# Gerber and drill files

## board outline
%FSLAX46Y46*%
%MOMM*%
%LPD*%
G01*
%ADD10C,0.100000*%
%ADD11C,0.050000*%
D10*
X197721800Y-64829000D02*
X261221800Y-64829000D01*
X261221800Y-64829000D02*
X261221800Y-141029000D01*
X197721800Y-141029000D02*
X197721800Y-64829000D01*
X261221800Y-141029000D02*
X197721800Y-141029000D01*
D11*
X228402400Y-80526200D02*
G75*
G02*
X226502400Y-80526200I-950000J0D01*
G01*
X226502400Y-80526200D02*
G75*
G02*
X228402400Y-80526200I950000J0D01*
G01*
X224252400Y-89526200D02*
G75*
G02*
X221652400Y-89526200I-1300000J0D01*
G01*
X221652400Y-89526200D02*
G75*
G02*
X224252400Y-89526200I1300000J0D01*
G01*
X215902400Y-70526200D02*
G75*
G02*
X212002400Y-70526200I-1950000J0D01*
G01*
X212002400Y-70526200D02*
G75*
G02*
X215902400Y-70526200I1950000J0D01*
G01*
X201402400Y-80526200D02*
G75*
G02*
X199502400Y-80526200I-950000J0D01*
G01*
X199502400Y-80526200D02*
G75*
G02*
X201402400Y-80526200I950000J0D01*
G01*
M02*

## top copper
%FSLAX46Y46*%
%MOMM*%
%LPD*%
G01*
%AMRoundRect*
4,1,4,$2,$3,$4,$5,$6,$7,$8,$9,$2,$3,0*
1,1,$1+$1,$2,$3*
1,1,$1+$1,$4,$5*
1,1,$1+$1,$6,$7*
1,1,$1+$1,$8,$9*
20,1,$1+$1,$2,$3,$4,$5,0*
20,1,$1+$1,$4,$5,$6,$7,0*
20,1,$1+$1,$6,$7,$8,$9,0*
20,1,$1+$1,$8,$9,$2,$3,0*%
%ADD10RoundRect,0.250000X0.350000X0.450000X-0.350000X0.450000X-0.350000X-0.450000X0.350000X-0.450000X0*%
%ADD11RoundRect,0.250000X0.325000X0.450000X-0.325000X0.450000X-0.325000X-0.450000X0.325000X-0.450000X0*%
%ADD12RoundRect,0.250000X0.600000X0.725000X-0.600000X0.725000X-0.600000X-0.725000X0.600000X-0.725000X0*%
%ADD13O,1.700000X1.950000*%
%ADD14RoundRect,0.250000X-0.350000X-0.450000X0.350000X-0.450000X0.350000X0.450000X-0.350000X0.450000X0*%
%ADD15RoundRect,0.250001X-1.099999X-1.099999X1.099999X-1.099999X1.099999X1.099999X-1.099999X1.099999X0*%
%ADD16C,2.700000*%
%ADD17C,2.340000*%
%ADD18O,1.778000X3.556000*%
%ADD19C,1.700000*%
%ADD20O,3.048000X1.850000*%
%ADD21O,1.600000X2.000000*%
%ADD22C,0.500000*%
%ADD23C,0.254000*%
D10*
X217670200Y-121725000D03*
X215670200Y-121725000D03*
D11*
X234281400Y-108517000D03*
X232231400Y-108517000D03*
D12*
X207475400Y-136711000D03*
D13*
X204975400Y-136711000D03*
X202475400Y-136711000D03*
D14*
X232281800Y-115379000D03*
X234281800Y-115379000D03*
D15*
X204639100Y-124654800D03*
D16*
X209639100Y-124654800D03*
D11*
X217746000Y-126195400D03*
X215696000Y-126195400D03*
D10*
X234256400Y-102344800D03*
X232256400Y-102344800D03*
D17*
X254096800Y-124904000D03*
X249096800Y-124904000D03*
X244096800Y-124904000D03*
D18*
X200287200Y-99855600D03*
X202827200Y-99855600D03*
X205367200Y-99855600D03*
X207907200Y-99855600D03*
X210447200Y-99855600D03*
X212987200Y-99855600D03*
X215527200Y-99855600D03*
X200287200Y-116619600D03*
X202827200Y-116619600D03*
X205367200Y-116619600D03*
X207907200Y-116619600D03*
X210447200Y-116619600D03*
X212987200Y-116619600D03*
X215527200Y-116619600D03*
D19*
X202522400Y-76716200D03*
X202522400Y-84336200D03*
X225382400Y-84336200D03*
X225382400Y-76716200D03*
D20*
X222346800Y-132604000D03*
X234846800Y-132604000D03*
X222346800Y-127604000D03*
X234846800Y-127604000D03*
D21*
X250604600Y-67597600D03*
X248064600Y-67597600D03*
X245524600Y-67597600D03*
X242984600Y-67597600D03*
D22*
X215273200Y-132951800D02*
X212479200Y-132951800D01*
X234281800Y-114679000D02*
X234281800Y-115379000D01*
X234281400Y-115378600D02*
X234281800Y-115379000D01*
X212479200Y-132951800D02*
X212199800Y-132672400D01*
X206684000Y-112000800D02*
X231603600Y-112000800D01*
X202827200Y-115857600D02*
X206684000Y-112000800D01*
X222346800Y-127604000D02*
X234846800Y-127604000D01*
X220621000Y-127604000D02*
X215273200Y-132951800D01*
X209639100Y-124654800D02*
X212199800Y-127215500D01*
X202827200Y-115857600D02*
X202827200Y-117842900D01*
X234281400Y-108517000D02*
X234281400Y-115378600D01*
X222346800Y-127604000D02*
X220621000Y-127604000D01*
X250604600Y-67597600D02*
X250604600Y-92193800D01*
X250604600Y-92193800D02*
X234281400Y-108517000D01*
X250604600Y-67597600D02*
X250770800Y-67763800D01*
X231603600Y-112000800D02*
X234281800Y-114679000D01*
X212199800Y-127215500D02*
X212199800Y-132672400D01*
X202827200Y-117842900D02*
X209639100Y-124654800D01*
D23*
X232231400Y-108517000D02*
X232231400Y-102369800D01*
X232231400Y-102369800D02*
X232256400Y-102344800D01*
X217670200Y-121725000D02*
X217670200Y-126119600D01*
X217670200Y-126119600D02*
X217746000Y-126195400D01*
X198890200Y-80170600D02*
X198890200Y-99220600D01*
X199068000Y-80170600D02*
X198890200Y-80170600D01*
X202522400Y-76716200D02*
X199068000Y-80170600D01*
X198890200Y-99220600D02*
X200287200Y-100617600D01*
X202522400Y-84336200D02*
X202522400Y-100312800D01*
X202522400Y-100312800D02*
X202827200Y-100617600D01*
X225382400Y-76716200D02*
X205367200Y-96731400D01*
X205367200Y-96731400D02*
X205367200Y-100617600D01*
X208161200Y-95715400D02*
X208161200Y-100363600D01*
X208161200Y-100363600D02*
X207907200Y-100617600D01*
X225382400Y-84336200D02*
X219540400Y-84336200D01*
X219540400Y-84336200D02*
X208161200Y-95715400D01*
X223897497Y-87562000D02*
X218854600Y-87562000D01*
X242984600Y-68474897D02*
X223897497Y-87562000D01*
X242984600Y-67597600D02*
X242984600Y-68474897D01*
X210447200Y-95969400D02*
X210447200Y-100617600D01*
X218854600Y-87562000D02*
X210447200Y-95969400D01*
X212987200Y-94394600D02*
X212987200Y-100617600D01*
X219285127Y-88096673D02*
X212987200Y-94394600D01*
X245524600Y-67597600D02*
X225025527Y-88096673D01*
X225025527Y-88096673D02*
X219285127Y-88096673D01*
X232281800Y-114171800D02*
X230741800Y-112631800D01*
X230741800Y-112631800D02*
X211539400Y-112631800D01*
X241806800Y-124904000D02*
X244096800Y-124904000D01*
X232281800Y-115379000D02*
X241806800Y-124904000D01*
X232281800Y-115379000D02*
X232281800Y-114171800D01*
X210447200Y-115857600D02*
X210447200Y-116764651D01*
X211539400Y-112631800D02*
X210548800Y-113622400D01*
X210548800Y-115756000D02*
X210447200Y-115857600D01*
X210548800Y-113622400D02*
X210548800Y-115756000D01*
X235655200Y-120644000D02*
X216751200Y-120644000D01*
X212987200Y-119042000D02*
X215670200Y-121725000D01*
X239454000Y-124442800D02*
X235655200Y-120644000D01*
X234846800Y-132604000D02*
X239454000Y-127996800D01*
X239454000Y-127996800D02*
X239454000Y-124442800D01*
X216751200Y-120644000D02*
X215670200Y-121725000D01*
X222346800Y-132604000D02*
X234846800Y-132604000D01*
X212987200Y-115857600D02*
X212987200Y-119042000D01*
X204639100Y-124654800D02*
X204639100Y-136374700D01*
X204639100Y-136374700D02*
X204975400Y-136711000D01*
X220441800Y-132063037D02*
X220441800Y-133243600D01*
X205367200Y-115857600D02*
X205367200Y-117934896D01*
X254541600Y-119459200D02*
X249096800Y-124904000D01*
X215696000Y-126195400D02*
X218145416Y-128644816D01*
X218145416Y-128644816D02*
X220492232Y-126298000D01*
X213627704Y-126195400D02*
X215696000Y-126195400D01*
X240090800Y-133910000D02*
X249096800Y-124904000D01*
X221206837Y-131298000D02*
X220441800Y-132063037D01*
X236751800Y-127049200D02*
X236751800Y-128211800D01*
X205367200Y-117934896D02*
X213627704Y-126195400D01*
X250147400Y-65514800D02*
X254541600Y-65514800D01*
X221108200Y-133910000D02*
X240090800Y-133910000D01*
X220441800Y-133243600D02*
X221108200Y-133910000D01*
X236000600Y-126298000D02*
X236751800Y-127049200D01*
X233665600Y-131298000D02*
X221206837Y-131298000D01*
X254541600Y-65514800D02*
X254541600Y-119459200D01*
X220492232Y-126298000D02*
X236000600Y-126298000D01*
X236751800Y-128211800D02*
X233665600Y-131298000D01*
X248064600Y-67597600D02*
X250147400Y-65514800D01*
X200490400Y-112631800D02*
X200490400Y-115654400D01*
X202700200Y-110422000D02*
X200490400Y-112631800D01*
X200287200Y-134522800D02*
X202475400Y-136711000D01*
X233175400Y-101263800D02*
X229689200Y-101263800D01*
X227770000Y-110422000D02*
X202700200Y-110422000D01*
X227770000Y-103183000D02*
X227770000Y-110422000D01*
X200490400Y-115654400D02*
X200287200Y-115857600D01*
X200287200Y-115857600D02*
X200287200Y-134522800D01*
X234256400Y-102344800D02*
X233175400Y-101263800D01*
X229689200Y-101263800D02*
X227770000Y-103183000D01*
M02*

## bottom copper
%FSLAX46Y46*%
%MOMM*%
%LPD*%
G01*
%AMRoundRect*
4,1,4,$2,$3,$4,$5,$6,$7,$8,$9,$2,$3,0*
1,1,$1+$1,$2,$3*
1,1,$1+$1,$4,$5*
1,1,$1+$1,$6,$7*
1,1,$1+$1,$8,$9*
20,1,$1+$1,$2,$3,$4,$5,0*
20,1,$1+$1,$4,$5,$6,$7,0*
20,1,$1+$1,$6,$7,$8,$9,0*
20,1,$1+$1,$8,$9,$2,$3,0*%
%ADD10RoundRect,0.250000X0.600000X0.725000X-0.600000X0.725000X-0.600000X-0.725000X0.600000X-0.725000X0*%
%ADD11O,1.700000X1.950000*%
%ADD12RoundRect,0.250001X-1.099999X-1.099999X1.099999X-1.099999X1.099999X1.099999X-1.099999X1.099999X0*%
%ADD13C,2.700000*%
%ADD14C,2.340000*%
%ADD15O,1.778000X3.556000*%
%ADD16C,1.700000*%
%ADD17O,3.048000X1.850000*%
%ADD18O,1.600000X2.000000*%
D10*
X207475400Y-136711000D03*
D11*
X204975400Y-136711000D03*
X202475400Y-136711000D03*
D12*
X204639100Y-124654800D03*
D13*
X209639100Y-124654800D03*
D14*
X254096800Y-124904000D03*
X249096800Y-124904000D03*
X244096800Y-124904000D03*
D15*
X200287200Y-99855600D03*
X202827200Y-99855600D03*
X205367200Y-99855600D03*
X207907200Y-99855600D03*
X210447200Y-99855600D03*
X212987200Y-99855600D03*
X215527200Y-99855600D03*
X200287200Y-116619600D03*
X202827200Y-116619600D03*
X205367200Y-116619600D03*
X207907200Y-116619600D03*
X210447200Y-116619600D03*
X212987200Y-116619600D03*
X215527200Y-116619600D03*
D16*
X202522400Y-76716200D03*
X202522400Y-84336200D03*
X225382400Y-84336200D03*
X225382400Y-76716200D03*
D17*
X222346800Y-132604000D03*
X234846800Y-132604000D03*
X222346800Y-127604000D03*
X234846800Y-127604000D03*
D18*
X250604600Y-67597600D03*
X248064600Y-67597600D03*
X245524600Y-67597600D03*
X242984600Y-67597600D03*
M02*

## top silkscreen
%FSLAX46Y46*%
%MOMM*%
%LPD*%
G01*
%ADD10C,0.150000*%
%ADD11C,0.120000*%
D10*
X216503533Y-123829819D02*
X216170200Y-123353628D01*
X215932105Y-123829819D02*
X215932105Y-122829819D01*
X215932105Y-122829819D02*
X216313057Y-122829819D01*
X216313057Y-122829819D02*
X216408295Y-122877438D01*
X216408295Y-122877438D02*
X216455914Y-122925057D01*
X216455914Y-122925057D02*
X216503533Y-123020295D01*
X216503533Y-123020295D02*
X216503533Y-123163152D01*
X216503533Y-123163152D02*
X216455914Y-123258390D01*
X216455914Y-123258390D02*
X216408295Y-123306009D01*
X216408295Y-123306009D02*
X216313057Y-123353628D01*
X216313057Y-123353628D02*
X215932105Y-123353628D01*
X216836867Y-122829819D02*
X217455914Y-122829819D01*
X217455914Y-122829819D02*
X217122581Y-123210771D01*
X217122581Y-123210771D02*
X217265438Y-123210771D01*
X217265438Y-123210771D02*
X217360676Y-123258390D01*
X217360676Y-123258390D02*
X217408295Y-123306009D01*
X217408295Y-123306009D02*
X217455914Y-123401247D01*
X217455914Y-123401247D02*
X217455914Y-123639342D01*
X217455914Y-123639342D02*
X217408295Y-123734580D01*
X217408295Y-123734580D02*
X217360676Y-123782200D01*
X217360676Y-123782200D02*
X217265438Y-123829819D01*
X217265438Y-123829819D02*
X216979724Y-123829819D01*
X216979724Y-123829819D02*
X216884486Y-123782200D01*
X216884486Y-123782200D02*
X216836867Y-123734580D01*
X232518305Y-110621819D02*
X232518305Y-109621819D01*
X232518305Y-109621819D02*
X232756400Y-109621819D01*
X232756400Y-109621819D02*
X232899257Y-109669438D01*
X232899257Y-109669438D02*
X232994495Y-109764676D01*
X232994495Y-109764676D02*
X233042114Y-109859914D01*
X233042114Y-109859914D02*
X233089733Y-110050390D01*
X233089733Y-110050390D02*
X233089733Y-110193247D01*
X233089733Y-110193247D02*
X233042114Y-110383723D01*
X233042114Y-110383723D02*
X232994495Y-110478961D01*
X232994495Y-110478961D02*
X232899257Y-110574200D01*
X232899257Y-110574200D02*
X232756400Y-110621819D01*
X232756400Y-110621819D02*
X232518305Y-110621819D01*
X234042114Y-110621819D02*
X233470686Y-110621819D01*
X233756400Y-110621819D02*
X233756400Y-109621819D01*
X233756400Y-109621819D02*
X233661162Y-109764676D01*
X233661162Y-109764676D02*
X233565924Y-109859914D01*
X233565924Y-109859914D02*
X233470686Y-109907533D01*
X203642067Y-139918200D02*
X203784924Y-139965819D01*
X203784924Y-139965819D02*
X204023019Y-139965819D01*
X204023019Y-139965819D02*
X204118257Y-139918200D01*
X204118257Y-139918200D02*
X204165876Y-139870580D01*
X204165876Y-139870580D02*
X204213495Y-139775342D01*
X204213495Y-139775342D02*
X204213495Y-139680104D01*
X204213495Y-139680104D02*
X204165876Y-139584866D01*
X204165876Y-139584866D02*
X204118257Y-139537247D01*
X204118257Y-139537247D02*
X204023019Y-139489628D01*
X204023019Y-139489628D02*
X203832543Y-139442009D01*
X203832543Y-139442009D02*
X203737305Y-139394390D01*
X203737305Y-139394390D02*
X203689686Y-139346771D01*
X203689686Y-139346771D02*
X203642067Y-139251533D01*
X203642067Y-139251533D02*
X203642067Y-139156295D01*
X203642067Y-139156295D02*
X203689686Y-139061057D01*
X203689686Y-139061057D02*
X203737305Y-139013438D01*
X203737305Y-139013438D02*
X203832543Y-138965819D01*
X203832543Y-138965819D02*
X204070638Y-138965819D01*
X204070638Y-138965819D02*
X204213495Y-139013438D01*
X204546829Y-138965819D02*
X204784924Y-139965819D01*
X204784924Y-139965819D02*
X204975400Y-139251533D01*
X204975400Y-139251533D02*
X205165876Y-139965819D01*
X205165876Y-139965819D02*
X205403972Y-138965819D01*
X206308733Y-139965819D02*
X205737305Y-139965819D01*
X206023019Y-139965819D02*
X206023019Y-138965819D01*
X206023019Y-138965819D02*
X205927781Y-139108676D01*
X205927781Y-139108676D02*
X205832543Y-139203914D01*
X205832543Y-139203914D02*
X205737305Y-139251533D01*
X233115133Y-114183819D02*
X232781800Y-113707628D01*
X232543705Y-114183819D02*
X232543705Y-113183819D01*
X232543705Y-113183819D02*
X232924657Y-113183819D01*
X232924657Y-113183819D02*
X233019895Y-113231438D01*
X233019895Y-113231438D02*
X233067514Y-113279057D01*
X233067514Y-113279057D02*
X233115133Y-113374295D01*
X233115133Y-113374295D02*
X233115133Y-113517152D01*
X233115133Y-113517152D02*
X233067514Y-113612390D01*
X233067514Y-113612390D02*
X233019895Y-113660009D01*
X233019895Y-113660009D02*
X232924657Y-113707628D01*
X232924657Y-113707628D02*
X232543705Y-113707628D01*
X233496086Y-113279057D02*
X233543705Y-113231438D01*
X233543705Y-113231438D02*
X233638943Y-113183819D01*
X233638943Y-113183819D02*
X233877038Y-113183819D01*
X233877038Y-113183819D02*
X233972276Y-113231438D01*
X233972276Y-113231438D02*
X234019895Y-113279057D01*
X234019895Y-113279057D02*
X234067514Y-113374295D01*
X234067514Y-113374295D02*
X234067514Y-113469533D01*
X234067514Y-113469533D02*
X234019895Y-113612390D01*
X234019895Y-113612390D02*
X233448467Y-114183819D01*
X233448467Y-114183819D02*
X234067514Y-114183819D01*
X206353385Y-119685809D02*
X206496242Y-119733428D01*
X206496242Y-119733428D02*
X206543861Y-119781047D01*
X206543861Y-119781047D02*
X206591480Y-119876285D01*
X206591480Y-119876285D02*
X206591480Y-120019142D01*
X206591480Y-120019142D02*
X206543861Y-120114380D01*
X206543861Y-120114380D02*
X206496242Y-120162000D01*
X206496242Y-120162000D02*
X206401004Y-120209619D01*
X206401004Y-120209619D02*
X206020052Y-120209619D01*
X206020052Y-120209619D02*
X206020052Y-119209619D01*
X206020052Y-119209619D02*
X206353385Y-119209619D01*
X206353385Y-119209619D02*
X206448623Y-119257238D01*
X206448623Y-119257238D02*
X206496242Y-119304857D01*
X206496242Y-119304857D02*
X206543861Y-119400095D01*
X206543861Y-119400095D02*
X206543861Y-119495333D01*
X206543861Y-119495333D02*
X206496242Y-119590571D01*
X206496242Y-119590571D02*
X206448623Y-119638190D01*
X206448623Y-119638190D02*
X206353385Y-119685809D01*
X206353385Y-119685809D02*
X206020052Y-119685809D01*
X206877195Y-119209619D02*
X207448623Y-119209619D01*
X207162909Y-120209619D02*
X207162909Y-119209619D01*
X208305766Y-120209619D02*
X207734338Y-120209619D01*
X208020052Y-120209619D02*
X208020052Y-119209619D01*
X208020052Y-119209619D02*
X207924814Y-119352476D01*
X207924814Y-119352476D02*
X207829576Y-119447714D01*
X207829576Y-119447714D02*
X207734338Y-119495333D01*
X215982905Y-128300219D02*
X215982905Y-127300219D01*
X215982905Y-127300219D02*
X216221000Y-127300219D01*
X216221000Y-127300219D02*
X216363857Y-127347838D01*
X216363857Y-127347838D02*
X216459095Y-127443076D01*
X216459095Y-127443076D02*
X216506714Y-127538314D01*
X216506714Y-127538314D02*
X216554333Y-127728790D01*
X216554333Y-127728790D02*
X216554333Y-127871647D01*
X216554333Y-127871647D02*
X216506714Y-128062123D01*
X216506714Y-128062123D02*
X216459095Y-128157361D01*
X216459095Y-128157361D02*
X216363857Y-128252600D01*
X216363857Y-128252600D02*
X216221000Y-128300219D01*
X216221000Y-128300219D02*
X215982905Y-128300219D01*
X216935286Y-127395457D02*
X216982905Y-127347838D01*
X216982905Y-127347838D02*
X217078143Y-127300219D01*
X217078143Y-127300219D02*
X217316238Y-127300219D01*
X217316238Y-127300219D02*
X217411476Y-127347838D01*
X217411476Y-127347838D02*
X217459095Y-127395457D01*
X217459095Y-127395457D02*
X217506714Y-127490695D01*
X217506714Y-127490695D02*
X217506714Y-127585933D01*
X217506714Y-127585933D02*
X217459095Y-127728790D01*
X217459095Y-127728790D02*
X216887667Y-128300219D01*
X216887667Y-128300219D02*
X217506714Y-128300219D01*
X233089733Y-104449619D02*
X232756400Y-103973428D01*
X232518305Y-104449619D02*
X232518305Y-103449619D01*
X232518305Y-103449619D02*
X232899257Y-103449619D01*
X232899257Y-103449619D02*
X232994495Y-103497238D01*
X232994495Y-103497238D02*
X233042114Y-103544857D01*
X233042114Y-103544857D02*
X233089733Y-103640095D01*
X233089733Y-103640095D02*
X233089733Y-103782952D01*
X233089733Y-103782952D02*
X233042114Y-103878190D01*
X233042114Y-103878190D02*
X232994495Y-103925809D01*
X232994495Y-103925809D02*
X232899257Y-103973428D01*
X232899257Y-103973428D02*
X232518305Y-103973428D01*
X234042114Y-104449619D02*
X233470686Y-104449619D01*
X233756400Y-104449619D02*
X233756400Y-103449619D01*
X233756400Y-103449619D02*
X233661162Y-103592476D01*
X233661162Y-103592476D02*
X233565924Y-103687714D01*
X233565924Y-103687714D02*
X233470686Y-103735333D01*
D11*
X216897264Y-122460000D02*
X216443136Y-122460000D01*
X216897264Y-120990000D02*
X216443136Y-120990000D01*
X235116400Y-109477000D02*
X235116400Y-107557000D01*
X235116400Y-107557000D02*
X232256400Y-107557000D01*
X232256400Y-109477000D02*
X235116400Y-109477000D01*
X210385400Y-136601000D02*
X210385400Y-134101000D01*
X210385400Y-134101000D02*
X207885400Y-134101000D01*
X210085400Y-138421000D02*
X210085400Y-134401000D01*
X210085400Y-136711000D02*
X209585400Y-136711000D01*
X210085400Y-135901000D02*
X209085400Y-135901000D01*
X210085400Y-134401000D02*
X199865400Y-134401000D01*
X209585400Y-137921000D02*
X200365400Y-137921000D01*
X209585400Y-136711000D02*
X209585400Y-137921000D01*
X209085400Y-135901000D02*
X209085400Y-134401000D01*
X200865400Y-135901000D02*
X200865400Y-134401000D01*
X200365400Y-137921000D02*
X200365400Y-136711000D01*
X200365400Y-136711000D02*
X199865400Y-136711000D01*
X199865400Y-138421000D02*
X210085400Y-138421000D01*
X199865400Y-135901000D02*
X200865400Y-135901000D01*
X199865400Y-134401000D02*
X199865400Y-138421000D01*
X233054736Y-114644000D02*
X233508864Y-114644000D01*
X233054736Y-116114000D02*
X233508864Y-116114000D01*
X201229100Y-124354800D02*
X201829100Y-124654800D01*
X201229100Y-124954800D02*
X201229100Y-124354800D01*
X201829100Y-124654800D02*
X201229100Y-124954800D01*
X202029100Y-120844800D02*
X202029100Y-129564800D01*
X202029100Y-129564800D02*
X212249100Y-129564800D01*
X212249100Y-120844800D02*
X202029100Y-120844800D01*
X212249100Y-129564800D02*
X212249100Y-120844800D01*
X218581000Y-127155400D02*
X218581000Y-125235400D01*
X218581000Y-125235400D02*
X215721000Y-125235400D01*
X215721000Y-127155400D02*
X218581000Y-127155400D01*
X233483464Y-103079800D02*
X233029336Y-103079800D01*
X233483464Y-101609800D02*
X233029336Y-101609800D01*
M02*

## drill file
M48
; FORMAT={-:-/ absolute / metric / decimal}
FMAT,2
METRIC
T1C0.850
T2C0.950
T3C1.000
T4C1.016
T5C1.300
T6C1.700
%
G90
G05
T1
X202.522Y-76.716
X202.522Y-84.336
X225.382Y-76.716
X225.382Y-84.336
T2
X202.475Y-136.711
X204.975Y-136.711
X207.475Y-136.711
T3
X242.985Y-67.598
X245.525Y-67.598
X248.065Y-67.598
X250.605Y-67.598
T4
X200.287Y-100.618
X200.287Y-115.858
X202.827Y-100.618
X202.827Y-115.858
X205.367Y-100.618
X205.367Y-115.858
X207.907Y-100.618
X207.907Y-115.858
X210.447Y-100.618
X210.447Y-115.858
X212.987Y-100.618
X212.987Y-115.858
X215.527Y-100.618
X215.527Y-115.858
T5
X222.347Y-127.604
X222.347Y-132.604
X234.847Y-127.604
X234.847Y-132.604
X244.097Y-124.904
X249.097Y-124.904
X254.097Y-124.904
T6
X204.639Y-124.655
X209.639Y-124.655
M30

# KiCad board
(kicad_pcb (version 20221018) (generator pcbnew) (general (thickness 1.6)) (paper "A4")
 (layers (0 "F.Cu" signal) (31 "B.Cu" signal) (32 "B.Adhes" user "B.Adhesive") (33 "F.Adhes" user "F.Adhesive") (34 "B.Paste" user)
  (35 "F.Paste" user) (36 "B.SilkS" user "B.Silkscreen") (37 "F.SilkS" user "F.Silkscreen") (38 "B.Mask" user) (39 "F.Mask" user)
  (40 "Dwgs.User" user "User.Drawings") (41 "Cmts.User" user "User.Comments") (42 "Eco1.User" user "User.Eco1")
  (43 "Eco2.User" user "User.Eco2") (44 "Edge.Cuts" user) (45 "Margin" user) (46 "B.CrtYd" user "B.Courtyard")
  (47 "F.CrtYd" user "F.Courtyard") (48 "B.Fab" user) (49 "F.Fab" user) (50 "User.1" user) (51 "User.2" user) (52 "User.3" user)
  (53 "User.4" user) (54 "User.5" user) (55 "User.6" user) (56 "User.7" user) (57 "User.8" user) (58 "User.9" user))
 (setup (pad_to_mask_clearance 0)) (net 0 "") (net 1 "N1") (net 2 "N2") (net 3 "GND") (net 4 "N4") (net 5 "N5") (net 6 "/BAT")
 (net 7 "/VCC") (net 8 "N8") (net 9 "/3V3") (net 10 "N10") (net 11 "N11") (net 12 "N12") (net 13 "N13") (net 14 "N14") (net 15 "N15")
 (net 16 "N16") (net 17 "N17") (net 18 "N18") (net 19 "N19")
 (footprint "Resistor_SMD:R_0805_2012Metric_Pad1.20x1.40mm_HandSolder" (layer "F.Cu") (at 216.6702 121.725 180)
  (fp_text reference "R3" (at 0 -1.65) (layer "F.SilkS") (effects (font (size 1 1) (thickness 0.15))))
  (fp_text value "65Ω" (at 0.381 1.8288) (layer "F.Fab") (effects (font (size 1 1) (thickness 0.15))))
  (fp_line (start -0.227064 -0.735) (end 0.227064 -0.735) (stroke (width 0.12) (type solid)) (layer "F.SilkS"))
  (fp_line (start -0.227064 0.735) (end 0.227064 0.735) (stroke (width 0.12) (type solid)) (layer "F.SilkS"))
  (pad "1" smd roundrect (at -1 0 180) (size 1.2 1.4) (layers "F.Cu" "F.Paste" "F.Mask") (roundrect_rratio 0.208333) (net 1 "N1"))
  (pad "2" smd roundrect (at 1 0 180) (size 1.2 1.4) (layers "F.Cu" "F.Paste" "F.Mask") (roundrect_rratio 0.208333) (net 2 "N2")))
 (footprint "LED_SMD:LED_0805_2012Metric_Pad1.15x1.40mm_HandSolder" (layer "F.Cu") (at 233.2564 108.517 180)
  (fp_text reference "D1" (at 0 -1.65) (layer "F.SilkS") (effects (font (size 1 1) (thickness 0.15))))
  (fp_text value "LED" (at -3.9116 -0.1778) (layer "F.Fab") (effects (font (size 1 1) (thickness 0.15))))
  (fp_line (start -1.86 -0.96) (end -1.86 0.96) (stroke (width 0.12) (type solid)) (layer "F.SilkS"))
  (fp_line (start -1.86 0.96) (end 1 0.96) (stroke (width 0.12) (type solid)) (layer "F.SilkS"))
  (fp_line (start 1 -0.96) (end -1.86 -0.96) (stroke (width 0.12) (type solid)) (layer "F.SilkS"))
  (pad "1" smd roundrect (at -1.025 0 180) (size 1.15 1.4) (layers "F.Cu" "F.Paste" "F.Mask") (roundrect_rratio 0.217391) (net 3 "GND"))
  (pad "2" smd roundrect (at 1.025 0 180) (size 1.15 1.4) (layers "F.Cu" "F.Paste" "F.Mask") (roundrect_rratio 0.217391) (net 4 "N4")))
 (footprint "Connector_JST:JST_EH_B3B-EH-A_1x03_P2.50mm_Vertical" (layer "F.Cu") (at 207.4754 136.711 180)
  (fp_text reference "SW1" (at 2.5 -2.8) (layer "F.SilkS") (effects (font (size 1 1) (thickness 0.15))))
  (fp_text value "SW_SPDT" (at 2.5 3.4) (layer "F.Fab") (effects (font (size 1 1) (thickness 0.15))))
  (fp_line (start -2.91 0.11) (end -2.91 2.61) (stroke (width 0.12) (type solid)) (layer "F.SilkS"))
  (fp_line (start -2.91 2.61) (end -0.41 2.61) (stroke (width 0.12) (type solid)) (layer "F.SilkS"))
  (fp_line (start -2.61 -1.71) (end -2.61 2.31) (stroke (width 0.12) (type solid)) (layer "F.SilkS"))
  (fp_line (start -2.61 0) (end -2.11 0) (stroke (width 0.12) (type solid)) (layer "F.SilkS"))
  (fp_line (start -2.61 0.81) (end -1.61 0.81) (stroke (width 0.12) (type solid)) (layer "F.SilkS"))
  (fp_line (start -2.61 2.31) (end 7.61 2.31) (stroke (width 0.12) (type solid)) (layer "F.SilkS"))
  (fp_line (start -2.11 -1.21) (end 7.11 -1.21) (stroke (width 0.12) (type solid)) (layer "F.SilkS"))
  (fp_line (start -2.11 0) (end -2.11 -1.21) (stroke (width 0.12) (type solid)) (layer "F.SilkS"))
  (fp_line (start -1.61 0.81) (end -1.61 2.31) (stroke (width 0.12) (type solid)) (layer "F.SilkS"))
  (fp_line (start 6.61 0.81) (end 6.61 2.31) (stroke (width 0.12) (type solid)) (layer "F.SilkS"))
  (fp_line (start 7.11 -1.21) (end 7.11 0) (stroke (width 0.12) (type solid)) (layer "F.SilkS"))
  (fp_line (start 7.11 0) (end 7.61 0) (stroke (width 0.12) (type solid)) (layer "F.SilkS"))
  (fp_line (start 7.61 -1.71) (end -2.61 -1.71) (stroke (width 0.12) (type solid)) (layer "F.SilkS"))
  (fp_line (start 7.61 0.81) (end 6.61 0.81) (stroke (width 0.12) (type solid)) (layer "F.SilkS"))
  (fp_line (start 7.61 2.31) (end 7.61 -1.71) (stroke (width 0.12) (type solid)) (layer "F.SilkS"))
  (pad "1" thru_hole roundrect (at 0 0 180) (size 1.7 1.95) (drill 0.95) (layers "*.Cu" "*.Mask") (roundrect_rratio 0.147059) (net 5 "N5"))
  (pad "2" thru_hole oval (at 2.5 0 180) (size 1.7 1.95) (drill 0.95) (layers "*.Cu" "*.Mask") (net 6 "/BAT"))
  (pad "3" thru_hole oval (at 5 0 180) (size 1.7 1.95) (drill 0.95) (layers "*.Cu" "*.Mask") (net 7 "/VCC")))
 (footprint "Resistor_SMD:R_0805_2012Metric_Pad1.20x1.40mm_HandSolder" (layer "F.Cu") (at 233.2818 115.379)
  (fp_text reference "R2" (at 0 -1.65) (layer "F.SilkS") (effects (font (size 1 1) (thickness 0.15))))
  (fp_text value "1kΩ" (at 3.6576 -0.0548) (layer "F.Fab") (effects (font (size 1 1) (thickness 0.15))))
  (fp_line (start -0.227064 -0.735) (end 0.227064 -0.735) (stroke (width 0.12) (type solid)) (layer "F.SilkS"))
  (fp_line (start -0.227064 0.735) (end 0.227064 0.735) (stroke (width 0.12) (type solid)) (layer "F.SilkS"))
  (pad "1" smd roundrect (at -1 0) (size 1.2 1.4) (layers "F.Cu" "F.Paste" "F.Mask") (roundrect_rratio 0.208333) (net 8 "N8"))
  (pad "2" smd roundrect (at 1 0) (size 1.2 1.4) (layers "F.Cu" "F.Paste" "F.Mask") (roundrect_rratio 0.208333) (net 3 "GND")))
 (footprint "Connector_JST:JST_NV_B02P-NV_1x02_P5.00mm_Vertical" (layer "F.Cu") (at 204.6391 124.6548)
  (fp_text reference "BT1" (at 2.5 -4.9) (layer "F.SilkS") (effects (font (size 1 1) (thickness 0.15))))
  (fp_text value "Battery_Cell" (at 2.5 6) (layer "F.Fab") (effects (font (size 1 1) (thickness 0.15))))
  (fp_line (start -3.41 -0.3) (end -2.81 0) (stroke (width 0.12) (type solid)) (layer "F.SilkS"))
  (fp_line (start -3.41 0.3) (end -3.41 -0.3) (stroke (width 0.12) (type solid)) (layer "F.SilkS"))
  (fp_line (start -2.81 0) (end -3.41 0.3) (stroke (width 0.12) (type solid)) (layer "F.SilkS"))
  (fp_line (start -2.61 -3.81) (end -2.61 4.91) (stroke (width 0.12) (type solid)) (layer "F.SilkS"))
  (fp_line (start -2.61 4.91) (end 7.61 4.91) (stroke (width 0.12) (type solid)) (layer "F.SilkS"))
  (fp_line (start 7.61 -3.81) (end -2.61 -3.81) (stroke (width 0.12) (type solid)) (layer "F.SilkS"))
  (fp_line (start 7.61 4.91) (end 7.61 -3.81) (stroke (width 0.12) (type solid)) (layer "F.SilkS"))
  (pad "1" thru_hole roundrect (at 0 0) (size 2.7 2.7) (drill 1.7) (layers "*.Cu" "*.Mask") (roundrect_rratio 0.092593) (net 6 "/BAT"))
  (pad "2" thru_hole circle (at 5 0) (size 2.7 2.7) (drill 1.7) (layers "*.Cu" "*.Mask") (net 3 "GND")))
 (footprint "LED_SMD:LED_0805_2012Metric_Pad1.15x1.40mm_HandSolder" (layer "F.Cu") (at 216.721 126.1954 180)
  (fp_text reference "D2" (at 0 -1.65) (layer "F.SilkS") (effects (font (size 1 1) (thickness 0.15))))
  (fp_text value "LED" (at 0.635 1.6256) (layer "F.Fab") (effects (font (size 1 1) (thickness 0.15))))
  (fp_line (start -1.86 -0.96) (end -1.86 0.96) (stroke (width 0.12) (type solid)) (layer "F.SilkS"))
  (fp_line (start -1.86 0.96) (end 1 0.96) (stroke (width 0.12) (type solid)) (layer "F.SilkS"))
  (fp_line (start 1 -0.96) (end -1.86 -0.96) (stroke (width 0.12) (type solid)) (layer "F.SilkS"))
  (pad "1" smd roundrect (at -1.025 0 180) (size 1.15 1.4) (layers "F.Cu" "F.Paste" "F.Mask") (roundrect_rratio 0.217391) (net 1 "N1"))
  (pad "2" smd roundrect (at 1.025 0 180) (size 1.15 1.4) (layers "F.Cu" "F.Paste" "F.Mask") (roundrect_rratio 0.217391) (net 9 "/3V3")))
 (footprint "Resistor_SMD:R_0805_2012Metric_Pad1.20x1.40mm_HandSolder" (layer "F.Cu") (at 233.2564 102.3448 180)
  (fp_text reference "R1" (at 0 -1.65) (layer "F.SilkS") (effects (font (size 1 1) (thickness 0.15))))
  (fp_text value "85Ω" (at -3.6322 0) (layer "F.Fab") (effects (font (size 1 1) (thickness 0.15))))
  (fp_line (start -0.227064 -0.735) (end 0.227064 -0.735) (stroke (width 0.12) (type solid)) (layer "F.SilkS"))
  (fp_line (start -0.227064 0.735) (end 0.227064 0.735) (stroke (width 0.12) (type solid)) (layer "F.SilkS"))
  (pad "1" smd roundrect (at -1 0 180) (size 1.2 1.4) (layers "F.Cu" "F.Paste" "F.Mask") (roundrect_rratio 0.208333) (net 7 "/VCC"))
  (pad "2" smd roundrect (at 1 0 180) (size 1.2 1.4) (layers "F.Cu" "F.Paste" "F.Mask") (roundrect_rratio 0.208333) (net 4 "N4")))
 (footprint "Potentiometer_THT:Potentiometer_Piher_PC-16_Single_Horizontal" (layer "B.Cu") (at 254.0968 124.904 -90)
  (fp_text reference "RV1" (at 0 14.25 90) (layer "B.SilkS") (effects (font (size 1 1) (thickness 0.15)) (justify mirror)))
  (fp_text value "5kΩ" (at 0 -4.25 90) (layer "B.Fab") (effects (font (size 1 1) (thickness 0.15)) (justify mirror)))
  (pad "1" thru_hole circle (at 0 0 270) (size 2.34 2.34) (drill 1.3) (layers "*.Cu" "*.Mask") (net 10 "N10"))
  (pad "2" thru_hole circle (at 0 5 270) (size 2.34 2.34) (drill 1.3) (layers "*.Cu" "*.Mask") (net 9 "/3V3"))
  (pad "3" thru_hole circle (at 0 10 270) (size 2.34 2.34) (drill 1.3) (layers "*.Cu" "*.Mask") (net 8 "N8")))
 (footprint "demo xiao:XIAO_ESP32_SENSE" (layer "B.Cu") (at 207.9072 108.2376 -90)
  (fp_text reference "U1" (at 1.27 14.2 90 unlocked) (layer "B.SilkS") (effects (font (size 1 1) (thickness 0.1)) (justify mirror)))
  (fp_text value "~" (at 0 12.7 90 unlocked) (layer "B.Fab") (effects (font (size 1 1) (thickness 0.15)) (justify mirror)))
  (pad "1" thru_hole oval (at -7.62 7.62 270) (size 3.556 1.778) (drill 1.016 (offset -0.762 0)) (layers "*.Cu" "*.Mask") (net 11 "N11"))
  (pad "2" thru_hole oval (at -7.62 5.08 270) (size 3.556 1.778) (drill 1.016 (offset -0.762 0)) (layers "*.Cu" "*.Mask") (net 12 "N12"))
  (pad "3" thru_hole oval (at -7.62 2.54 270) (size 3.556 1.778) (drill 1.016 (offset -0.762 0)) (layers "*.Cu" "*.Mask") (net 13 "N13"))
  (pad "4" thru_hole oval (at -7.62 0 270) (size 3.556 1.778) (drill 1.016 (offset -0.762 0)) (layers "*.Cu" "*.Mask") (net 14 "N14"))
  (pad "5" thru_hole oval (at -7.62 -2.54 270) (size 3.556 1.778) (drill 1.016 (offset -0.762 0)) (layers "*.Cu" "*.Mask") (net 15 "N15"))
  (pad "6" thru_hole oval (at -7.62 -5.08 270) (size 3.556 1.778) (drill 1.016 (offset -0.762 0)) (layers "*.Cu" "*.Mask") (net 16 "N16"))
  (pad "7" thru_hole oval (at -7.62 -7.62 270) (size 3.556 1.778) (drill 1.016 (offset -0.762 0)) (layers "*.Cu" "*.Mask") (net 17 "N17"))
  (pad "8" thru_hole oval (at 7.62 7.62 270) (size 3.556 1.778) (drill 1.016 (offset 0.762 0)) (layers "*.Cu" "*.Mask") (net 7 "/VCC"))
  (pad "9" thru_hole oval (at 7.62 5.08 270) (size 3.556 1.778) (drill 1.016 (offset 0.762 0)) (layers "*.Cu" "*.Mask") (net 3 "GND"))
  (pad "10" thru_hole oval (at 7.62 2.54 270) (size 3.556 1.778) (drill 1.016 (offset 0.762 0)) (layers "*.Cu" "*.Mask") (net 9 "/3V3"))
  (pad "11" thru_hole oval (at 7.62 0 270) (size 3.556 1.778) (drill 1.016 (offset 0.762 0)) (layers "*.Cu" "*.Mask") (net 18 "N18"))
  (pad "12" thru_hole oval (at 7.62 -2.54 270) (size 3.556 1.778) (drill 1.016 (offset 0.762 0)) (layers "*.Cu" "*.Mask") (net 8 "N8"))
  (pad "13" thru_hole oval (at 7.62 -5.08 270) (size 3.556 1.778) (drill 1.016 (offset 0.762 0)) (layers "*.Cu" "*.Mask") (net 2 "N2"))
  (pad "14" thru_hole oval (at 7.62 -7.62 270) (size 3.556 1.778) (drill 1.016 (offset 0.762 0)) (layers "*.Cu" "*.Mask") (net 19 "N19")))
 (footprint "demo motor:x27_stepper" (layer "B.Cu") (at 211.4124 90.6862 180)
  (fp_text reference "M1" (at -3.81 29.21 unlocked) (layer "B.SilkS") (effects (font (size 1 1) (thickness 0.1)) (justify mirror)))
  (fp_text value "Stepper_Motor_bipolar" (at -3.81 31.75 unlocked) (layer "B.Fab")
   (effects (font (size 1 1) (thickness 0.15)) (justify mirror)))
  (fp_circle (center -16.04 10.16) (end -15.09 10.16) (stroke (width 0.05) (type default)) (fill none) (layer "Edge.Cuts"))
  (fp_circle (center -11.54 1.16) (end -10.24 1.16) (stroke (width 0.05) (type default)) (fill none) (layer "Edge.Cuts"))
  (fp_circle (center -2.54 20.16) (end -0.59 20.16) (stroke (width 0.05) (type default)) (fill none) (layer "Edge.Cuts"))
  (fp_circle (center 10.96 10.16) (end 11.91 10.16) (stroke (width 0.05) (type default)) (fill none) (layer "Edge.Cuts"))
  (pad "1" thru_hole circle (at 8.89 13.97 180) (size 1.7 1.7) (drill 0.85) (layers "*.Cu" "*.Mask") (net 11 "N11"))
  (pad "2" thru_hole circle (at 8.89 6.35 180) (size 1.7 1.7) (drill 0.85) (layers "*.Cu" "*.Mask") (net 12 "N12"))
  (pad "3" thru_hole circle (at -13.97 6.35 180) (size 1.7 1.7) (drill 0.85) (layers "*.Cu" "*.Mask") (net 14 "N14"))
  (pad "4" thru_hole circle (at -13.97 13.97 180) (size 1.7 1.7) (drill 0.85) (layers "*.Cu" "*.Mask") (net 13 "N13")))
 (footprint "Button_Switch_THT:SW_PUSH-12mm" (layer "B.Cu") (at 222.3468 132.604)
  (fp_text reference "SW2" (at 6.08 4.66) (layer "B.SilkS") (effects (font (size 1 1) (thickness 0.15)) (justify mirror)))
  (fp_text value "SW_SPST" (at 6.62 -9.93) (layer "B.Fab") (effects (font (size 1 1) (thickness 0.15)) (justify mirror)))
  (pad "1" thru_hole oval (at 0 0) (size 3.048 1.85) (drill 1.3) (layers "*.Cu" "*.Mask") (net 2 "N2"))
  (pad "1" thru_hole oval (at 12.5 0) (size 3.048 1.85) (drill 1.3) (layers "*.Cu" "*.Mask") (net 2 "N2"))
  (pad "2" thru_hole oval (at 0 -5) (size 3.048 1.85) (drill 1.3) (layers "*.Cu" "*.Mask") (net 3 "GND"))
  (pad "2" thru_hole oval (at 12.5 -5) (size 3.048 1.85) (drill 1.3) (layers "*.Cu" "*.Mask") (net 3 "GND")))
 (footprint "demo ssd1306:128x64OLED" (layer "B.Cu") (at 246.9846 78.1976 180)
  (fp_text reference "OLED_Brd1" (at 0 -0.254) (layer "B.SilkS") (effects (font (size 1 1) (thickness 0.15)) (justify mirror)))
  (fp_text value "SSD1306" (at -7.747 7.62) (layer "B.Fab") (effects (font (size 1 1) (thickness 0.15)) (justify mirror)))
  (pad "1" thru_hole oval (at -3.62 10.6 90) (size 2 1.6) (drill 1) (layers "*.Cu" "*.Mask") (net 3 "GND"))
  (pad "2" thru_hole oval (at -1.08 10.6 90) (size 2 1.6) (drill 1) (layers "*.Cu" "*.Mask") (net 9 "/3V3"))
  (pad "3" thru_hole oval (at 1.46 10.6 90) (size 2 1.6) (drill 1) (layers "*.Cu" "*.Mask") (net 16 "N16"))
  (pad "4" thru_hole oval (at 4 10.6 90) (size 2 1.6) (drill 1) (layers "*.Cu" "*.Mask") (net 15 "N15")))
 (gr_line (start 197.7218 64.829) (end 261.2218 64.829) (stroke (width 0.1) (type default)) (layer "Edge.Cuts"))
 (gr_line (start 261.2218 64.829) (end 261.2218 141.029) (stroke (width 0.1) (type default)) (layer "Edge.Cuts"))
 (gr_line (start 197.7218 141.029) (end 197.7218 64.829) (stroke (width 0.1) (type default)) (layer "Edge.Cuts"))
 (gr_line (start 261.2218 141.029) (end 197.7218 141.029) (stroke (width 0.1) (type default)) (layer "Edge.Cuts"))
 (segment (start 215.2732 132.9518) (end 212.4792 132.9518) (width 0.5) (layer "F.Cu") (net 3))
 (segment (start 234.2818 114.679) (end 234.2818 115.379) (width 0.5) (layer "F.Cu") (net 3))
 (segment (start 234.2814 115.3786) (end 234.2818 115.379) (width 0.5) (layer "F.Cu") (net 3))
 (segment (start 212.4792 132.9518) (end 212.1998 132.6724) (width 0.5) (layer "F.Cu") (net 3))
 (segment (start 206.684 112.0008) (end 231.6036 112.0008) (width 0.5) (layer "F.Cu") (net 3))
 (segment (start 202.8272 115.8576) (end 206.684 112.0008) (width 0.5) (layer "F.Cu") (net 3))
 (segment (start 222.3468 127.604) (end 234.8468 127.604) (width 0.5) (layer "F.Cu") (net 3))
 (segment (start 220.621 127.604) (end 215.2732 132.9518) (width 0.5) (layer "F.Cu") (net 3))
 (segment (start 209.6391 124.6548) (end 212.1998 127.2155) (width 0.5) (layer "F.Cu") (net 3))
 (segment (start 202.8272 115.8576) (end 202.8272 117.8429) (width 0.5) (layer "F.Cu") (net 3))
 (segment (start 234.2814 108.517) (end 234.2814 115.3786) (width 0.5) (layer "F.Cu") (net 3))
 (segment (start 222.3468 127.604) (end 220.621 127.604) (width 0.5) (layer "F.Cu") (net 3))
 (segment (start 250.6046 67.5976) (end 250.6046 92.1938) (width 0.5) (layer "F.Cu") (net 3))
 (segment (start 250.6046 92.1938) (end 234.2814 108.517) (width 0.5) (layer "F.Cu") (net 3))
 (segment (start 250.6046 67.5976) (end 250.7708 67.7638) (width 0.5) (layer "F.Cu") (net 3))
 (segment (start 231.6036 112.0008) (end 234.2818 114.679) (width 0.5) (layer "F.Cu") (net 3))
 (segment (start 212.1998 127.2155) (end 212.1998 132.6724) (width 0.5) (layer "F.Cu") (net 3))
 (segment (start 202.8272 117.8429) (end 209.6391 124.6548) (width 0.5) (layer "F.Cu") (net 3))
 (segment (start 232.2314 108.517) (end 232.2314 102.3698) (width 0.254) (layer "F.Cu") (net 4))
 (segment (start 232.2314 102.3698) (end 232.2564 102.3448) (width 0.254) (layer "F.Cu") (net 4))
 (segment (start 217.6702 121.725) (end 217.6702 126.1196) (width 0.254) (layer "F.Cu") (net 1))
 (segment (start 217.6702 126.1196) (end 217.746 126.1954) (width 0.254) (layer "F.Cu") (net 1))
 (segment (start 198.8902 80.1706) (end 198.8902 99.2206) (width 0.254) (layer "F.Cu") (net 11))
 (segment (start 199.068 80.1706) (end 198.8902 80.1706) (width 0.254) (layer "F.Cu") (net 11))
 (segment (start 202.5224 76.7162) (end 199.068 80.1706) (width 0.254) (layer "F.Cu") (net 11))
 (segment (start 198.8902 99.2206) (end 200.2872 100.6176) (width 0.254) (layer "F.Cu") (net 11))
 (segment (start 202.5224 84.3362) (end 202.5224 100.3128) (width 0.254) (layer "F.Cu") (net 12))
 (segment (start 202.5224 100.3128) (end 202.8272 100.6176) (width 0.254) (layer "F.Cu") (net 12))
 (segment (start 225.3824 76.7162) (end 205.3672 96.7314) (width 0.254) (layer "F.Cu") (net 13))
 (segment (start 205.3672 96.7314) (end 205.3672 100.6176) (width 0.254) (layer "F.Cu") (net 13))
 (segment (start 208.1612 95.7154) (end 208.1612 100.3636) (width 0.254) (layer "F.Cu") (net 14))
 (segment (start 208.1612 100.3636) (end 207.9072 100.6176) (width 0.254) (layer "F.Cu") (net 14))
 (segment (start 225.3824 84.3362) (end 219.5404 84.3362) (width 0.254) (layer "F.Cu") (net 14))
 (segment (start 219.5404 84.3362) (end 208.1612 95.7154) (width 0.254) (layer "F.Cu") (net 14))
 (segment (start 223.897497 87.562) (end 218.8546 87.562) (width 0.254) (layer "F.Cu") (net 15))
 (segment (start 242.9846 68.474897) (end 223.897497 87.562) (width 0.254) (layer "F.Cu") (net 15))
 (segment (start 242.9846 67.5976) (end 242.9846 68.474897) (width 0.254) (layer "F.Cu") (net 15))
 (segment (start 210.4472 95.9694) (end 210.4472 100.6176) (width 0.254) (layer "F.Cu") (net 15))
 (segment (start 218.8546 87.562) (end 210.4472 95.9694) (width 0.254) (layer "F.Cu") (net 15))
 (segment (start 212.9872 94.3946) (end 212.9872 100.6176) (width 0.254) (layer "F.Cu") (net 16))
 (segment (start 219.285127 88.096673) (end 212.9872 94.3946) (width 0.254) (layer "F.Cu") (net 16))
 (segment (start 245.5246 67.5976) (end 225.025527 88.096673) (width 0.254) (layer "F.Cu") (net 16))
 (segment (start 225.025527 88.096673) (end 219.285127 88.096673) (width 0.254) (layer "F.Cu") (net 16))
 (segment (start 232.2818 114.1718) (end 230.7418 112.6318) (width 0.254) (layer "F.Cu") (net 8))
 (segment (start 230.7418 112.6318) (end 211.5394 112.6318) (width 0.254) (layer "F.Cu") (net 8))
 (segment (start 241.8068 124.904) (end 244.0968 124.904) (width 0.254) (layer "F.Cu") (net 8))
 (segment (start 232.2818 115.379) (end 241.8068 124.904) (width 0.254) (layer "F.Cu") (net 8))
 (segment (start 232.2818 115.379) (end 232.2818 114.1718) (width 0.254) (layer "F.Cu") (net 8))
 (segment (start 210.4472 115.8576) (end 210.4472 116.764651) (width 0.254) (layer "F.Cu") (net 8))
 (segment (start 211.5394 112.6318) (end 210.5488 113.6224) (width 0.254) (layer "F.Cu") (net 8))
 (segment (start 210.5488 115.756) (end 210.4472 115.8576) (width 0.254) (layer "F.Cu") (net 8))
 (segment (start 210.5488 113.6224) (end 210.5488 115.756) (width 0.254) (layer "F.Cu") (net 8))
 (segment (start 235.6552 120.644) (end 216.7512 120.644) (width 0.254) (layer "F.Cu") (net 2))
 (segment (start 212.9872 119.042) (end 215.6702 121.725) (width 0.254) (layer "F.Cu") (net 2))
 (segment (start 239.454 124.4428) (end 235.6552 120.644) (width 0.254) (layer "F.Cu") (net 2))
 (segment (start 234.8468 132.604) (end 239.454 127.9968) (width 0.254) (layer "F.Cu") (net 2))
 (segment (start 239.454 127.9968) (end 239.454 124.4428) (width 0.254) (layer "F.Cu") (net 2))
 (segment (start 216.7512 120.644) (end 215.6702 121.725) (width 0.254) (layer "F.Cu") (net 2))
 (segment (start 222.3468 132.604) (end 234.8468 132.604) (width 0.254) (layer "F.Cu") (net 2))
 (segment (start 212.9872 115.8576) (end 212.9872 119.042) (width 0.254) (layer "F.Cu") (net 2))
 (segment (start 204.6391 124.6548) (end 204.6391 136.3747) (width 0.254) (layer "F.Cu") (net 6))
 (segment (start 204.6391 136.3747) (end 204.9754 136.711) (width 0.254) (layer "F.Cu") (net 6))
 (segment (start 220.4418 132.063037) (end 220.4418 133.2436) (width 0.254) (layer "F.Cu") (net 9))
 (segment (start 205.3672 115.8576) (end 205.3672 117.934896) (width 0.254) (layer "F.Cu") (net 9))
 (segment (start 254.5416 119.4592) (end 249.0968 124.904) (width 0.254) (layer "F.Cu") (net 9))
 (segment (start 215.696 126.1954) (end 218.145416 128.644816) (width 0.254) (layer "F.Cu") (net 9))
 (segment (start 218.145416 128.644816) (end 220.492232 126.298) (width 0.254) (layer "F.Cu") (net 9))
 (segment (start 213.627704 126.1954) (end 215.696 126.1954) (width 0.254) (layer "F.Cu") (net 9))
 (segment (start 240.0908 133.91) (end 249.0968 124.904) (width 0.254) (layer "F.Cu") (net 9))
 (segment (start 221.206837 131.298) (end 220.4418 132.063037) (width 0.254) (layer "F.Cu") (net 9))
 (segment (start 236.7518 127.0492) (end 236.7518 128.2118) (width 0.254) (layer "F.Cu") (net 9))
 (segment (start 205.3672 117.934896) (end 213.627704 126.1954) (width 0.254) (layer "F.Cu") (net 9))
 (segment (start 250.1474 65.5148) (end 254.5416 65.5148) (width 0.254) (layer "F.Cu") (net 9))
 (segment (start 221.1082 133.91) (end 240.0908 133.91) (width 0.254) (layer "F.Cu") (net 9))
 (segment (start 220.4418 133.2436) (end 221.1082 133.91) (width 0.254) (layer "F.Cu") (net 9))
 (segment (start 236.0006 126.298) (end 236.7518 127.0492) (width 0.254) (layer "F.Cu") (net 9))
 (segment (start 233.6656 131.298) (end 221.206837 131.298) (width 0.254) (layer "F.Cu") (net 9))
 (segment (start 254.5416 65.5148) (end 254.5416 119.4592) (width 0.254) (layer "F.Cu") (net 9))
 (segment (start 220.492232 126.298) (end 236.0006 126.298) (width 0.254) (layer "F.Cu") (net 9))
 (segment (start 236.7518 128.2118) (end 233.6656 131.298) (width 0.254) (layer "F.Cu") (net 9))
 (segment (start 248.0646 67.5976) (end 250.1474 65.5148) (width 0.254) (layer "F.Cu") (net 9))
 (segment (start 200.4904 112.6318) (end 200.4904 115.6544) (width 0.254) (layer "F.Cu") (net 7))
 (segment (start 202.7002 110.422) (end 200.4904 112.6318) (width 0.254) (layer "F.Cu") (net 7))
 (segment (start 200.2872 134.5228) (end 202.4754 136.711) (width 0.254) (layer "F.Cu") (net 7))
 (segment (start 233.1754 101.2638) (end 229.6892 101.2638) (width 0.254) (layer "F.Cu") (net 7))
 (segment (start 227.77 110.422) (end 202.7002 110.422) (width 0.254) (layer "F.Cu") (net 7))
 (segment (start 227.77 103.183) (end 227.77 110.422) (width 0.254) (layer "F.Cu") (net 7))
 (segment (start 200.4904 115.6544) (end 200.2872 115.8576) (width 0.254) (layer "F.Cu") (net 7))
 (segment (start 200.2872 115.8576) (end 200.2872 134.5228) (width 0.254) (layer "F.Cu") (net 7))
 (segment (start 234.2564 102.3448) (end 233.1754 101.2638) (width 0.254) (layer "F.Cu") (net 7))
 (segment (start 229.6892 101.2638) (end 227.77 103.183) (width 0.254) (layer "F.Cu") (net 7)))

